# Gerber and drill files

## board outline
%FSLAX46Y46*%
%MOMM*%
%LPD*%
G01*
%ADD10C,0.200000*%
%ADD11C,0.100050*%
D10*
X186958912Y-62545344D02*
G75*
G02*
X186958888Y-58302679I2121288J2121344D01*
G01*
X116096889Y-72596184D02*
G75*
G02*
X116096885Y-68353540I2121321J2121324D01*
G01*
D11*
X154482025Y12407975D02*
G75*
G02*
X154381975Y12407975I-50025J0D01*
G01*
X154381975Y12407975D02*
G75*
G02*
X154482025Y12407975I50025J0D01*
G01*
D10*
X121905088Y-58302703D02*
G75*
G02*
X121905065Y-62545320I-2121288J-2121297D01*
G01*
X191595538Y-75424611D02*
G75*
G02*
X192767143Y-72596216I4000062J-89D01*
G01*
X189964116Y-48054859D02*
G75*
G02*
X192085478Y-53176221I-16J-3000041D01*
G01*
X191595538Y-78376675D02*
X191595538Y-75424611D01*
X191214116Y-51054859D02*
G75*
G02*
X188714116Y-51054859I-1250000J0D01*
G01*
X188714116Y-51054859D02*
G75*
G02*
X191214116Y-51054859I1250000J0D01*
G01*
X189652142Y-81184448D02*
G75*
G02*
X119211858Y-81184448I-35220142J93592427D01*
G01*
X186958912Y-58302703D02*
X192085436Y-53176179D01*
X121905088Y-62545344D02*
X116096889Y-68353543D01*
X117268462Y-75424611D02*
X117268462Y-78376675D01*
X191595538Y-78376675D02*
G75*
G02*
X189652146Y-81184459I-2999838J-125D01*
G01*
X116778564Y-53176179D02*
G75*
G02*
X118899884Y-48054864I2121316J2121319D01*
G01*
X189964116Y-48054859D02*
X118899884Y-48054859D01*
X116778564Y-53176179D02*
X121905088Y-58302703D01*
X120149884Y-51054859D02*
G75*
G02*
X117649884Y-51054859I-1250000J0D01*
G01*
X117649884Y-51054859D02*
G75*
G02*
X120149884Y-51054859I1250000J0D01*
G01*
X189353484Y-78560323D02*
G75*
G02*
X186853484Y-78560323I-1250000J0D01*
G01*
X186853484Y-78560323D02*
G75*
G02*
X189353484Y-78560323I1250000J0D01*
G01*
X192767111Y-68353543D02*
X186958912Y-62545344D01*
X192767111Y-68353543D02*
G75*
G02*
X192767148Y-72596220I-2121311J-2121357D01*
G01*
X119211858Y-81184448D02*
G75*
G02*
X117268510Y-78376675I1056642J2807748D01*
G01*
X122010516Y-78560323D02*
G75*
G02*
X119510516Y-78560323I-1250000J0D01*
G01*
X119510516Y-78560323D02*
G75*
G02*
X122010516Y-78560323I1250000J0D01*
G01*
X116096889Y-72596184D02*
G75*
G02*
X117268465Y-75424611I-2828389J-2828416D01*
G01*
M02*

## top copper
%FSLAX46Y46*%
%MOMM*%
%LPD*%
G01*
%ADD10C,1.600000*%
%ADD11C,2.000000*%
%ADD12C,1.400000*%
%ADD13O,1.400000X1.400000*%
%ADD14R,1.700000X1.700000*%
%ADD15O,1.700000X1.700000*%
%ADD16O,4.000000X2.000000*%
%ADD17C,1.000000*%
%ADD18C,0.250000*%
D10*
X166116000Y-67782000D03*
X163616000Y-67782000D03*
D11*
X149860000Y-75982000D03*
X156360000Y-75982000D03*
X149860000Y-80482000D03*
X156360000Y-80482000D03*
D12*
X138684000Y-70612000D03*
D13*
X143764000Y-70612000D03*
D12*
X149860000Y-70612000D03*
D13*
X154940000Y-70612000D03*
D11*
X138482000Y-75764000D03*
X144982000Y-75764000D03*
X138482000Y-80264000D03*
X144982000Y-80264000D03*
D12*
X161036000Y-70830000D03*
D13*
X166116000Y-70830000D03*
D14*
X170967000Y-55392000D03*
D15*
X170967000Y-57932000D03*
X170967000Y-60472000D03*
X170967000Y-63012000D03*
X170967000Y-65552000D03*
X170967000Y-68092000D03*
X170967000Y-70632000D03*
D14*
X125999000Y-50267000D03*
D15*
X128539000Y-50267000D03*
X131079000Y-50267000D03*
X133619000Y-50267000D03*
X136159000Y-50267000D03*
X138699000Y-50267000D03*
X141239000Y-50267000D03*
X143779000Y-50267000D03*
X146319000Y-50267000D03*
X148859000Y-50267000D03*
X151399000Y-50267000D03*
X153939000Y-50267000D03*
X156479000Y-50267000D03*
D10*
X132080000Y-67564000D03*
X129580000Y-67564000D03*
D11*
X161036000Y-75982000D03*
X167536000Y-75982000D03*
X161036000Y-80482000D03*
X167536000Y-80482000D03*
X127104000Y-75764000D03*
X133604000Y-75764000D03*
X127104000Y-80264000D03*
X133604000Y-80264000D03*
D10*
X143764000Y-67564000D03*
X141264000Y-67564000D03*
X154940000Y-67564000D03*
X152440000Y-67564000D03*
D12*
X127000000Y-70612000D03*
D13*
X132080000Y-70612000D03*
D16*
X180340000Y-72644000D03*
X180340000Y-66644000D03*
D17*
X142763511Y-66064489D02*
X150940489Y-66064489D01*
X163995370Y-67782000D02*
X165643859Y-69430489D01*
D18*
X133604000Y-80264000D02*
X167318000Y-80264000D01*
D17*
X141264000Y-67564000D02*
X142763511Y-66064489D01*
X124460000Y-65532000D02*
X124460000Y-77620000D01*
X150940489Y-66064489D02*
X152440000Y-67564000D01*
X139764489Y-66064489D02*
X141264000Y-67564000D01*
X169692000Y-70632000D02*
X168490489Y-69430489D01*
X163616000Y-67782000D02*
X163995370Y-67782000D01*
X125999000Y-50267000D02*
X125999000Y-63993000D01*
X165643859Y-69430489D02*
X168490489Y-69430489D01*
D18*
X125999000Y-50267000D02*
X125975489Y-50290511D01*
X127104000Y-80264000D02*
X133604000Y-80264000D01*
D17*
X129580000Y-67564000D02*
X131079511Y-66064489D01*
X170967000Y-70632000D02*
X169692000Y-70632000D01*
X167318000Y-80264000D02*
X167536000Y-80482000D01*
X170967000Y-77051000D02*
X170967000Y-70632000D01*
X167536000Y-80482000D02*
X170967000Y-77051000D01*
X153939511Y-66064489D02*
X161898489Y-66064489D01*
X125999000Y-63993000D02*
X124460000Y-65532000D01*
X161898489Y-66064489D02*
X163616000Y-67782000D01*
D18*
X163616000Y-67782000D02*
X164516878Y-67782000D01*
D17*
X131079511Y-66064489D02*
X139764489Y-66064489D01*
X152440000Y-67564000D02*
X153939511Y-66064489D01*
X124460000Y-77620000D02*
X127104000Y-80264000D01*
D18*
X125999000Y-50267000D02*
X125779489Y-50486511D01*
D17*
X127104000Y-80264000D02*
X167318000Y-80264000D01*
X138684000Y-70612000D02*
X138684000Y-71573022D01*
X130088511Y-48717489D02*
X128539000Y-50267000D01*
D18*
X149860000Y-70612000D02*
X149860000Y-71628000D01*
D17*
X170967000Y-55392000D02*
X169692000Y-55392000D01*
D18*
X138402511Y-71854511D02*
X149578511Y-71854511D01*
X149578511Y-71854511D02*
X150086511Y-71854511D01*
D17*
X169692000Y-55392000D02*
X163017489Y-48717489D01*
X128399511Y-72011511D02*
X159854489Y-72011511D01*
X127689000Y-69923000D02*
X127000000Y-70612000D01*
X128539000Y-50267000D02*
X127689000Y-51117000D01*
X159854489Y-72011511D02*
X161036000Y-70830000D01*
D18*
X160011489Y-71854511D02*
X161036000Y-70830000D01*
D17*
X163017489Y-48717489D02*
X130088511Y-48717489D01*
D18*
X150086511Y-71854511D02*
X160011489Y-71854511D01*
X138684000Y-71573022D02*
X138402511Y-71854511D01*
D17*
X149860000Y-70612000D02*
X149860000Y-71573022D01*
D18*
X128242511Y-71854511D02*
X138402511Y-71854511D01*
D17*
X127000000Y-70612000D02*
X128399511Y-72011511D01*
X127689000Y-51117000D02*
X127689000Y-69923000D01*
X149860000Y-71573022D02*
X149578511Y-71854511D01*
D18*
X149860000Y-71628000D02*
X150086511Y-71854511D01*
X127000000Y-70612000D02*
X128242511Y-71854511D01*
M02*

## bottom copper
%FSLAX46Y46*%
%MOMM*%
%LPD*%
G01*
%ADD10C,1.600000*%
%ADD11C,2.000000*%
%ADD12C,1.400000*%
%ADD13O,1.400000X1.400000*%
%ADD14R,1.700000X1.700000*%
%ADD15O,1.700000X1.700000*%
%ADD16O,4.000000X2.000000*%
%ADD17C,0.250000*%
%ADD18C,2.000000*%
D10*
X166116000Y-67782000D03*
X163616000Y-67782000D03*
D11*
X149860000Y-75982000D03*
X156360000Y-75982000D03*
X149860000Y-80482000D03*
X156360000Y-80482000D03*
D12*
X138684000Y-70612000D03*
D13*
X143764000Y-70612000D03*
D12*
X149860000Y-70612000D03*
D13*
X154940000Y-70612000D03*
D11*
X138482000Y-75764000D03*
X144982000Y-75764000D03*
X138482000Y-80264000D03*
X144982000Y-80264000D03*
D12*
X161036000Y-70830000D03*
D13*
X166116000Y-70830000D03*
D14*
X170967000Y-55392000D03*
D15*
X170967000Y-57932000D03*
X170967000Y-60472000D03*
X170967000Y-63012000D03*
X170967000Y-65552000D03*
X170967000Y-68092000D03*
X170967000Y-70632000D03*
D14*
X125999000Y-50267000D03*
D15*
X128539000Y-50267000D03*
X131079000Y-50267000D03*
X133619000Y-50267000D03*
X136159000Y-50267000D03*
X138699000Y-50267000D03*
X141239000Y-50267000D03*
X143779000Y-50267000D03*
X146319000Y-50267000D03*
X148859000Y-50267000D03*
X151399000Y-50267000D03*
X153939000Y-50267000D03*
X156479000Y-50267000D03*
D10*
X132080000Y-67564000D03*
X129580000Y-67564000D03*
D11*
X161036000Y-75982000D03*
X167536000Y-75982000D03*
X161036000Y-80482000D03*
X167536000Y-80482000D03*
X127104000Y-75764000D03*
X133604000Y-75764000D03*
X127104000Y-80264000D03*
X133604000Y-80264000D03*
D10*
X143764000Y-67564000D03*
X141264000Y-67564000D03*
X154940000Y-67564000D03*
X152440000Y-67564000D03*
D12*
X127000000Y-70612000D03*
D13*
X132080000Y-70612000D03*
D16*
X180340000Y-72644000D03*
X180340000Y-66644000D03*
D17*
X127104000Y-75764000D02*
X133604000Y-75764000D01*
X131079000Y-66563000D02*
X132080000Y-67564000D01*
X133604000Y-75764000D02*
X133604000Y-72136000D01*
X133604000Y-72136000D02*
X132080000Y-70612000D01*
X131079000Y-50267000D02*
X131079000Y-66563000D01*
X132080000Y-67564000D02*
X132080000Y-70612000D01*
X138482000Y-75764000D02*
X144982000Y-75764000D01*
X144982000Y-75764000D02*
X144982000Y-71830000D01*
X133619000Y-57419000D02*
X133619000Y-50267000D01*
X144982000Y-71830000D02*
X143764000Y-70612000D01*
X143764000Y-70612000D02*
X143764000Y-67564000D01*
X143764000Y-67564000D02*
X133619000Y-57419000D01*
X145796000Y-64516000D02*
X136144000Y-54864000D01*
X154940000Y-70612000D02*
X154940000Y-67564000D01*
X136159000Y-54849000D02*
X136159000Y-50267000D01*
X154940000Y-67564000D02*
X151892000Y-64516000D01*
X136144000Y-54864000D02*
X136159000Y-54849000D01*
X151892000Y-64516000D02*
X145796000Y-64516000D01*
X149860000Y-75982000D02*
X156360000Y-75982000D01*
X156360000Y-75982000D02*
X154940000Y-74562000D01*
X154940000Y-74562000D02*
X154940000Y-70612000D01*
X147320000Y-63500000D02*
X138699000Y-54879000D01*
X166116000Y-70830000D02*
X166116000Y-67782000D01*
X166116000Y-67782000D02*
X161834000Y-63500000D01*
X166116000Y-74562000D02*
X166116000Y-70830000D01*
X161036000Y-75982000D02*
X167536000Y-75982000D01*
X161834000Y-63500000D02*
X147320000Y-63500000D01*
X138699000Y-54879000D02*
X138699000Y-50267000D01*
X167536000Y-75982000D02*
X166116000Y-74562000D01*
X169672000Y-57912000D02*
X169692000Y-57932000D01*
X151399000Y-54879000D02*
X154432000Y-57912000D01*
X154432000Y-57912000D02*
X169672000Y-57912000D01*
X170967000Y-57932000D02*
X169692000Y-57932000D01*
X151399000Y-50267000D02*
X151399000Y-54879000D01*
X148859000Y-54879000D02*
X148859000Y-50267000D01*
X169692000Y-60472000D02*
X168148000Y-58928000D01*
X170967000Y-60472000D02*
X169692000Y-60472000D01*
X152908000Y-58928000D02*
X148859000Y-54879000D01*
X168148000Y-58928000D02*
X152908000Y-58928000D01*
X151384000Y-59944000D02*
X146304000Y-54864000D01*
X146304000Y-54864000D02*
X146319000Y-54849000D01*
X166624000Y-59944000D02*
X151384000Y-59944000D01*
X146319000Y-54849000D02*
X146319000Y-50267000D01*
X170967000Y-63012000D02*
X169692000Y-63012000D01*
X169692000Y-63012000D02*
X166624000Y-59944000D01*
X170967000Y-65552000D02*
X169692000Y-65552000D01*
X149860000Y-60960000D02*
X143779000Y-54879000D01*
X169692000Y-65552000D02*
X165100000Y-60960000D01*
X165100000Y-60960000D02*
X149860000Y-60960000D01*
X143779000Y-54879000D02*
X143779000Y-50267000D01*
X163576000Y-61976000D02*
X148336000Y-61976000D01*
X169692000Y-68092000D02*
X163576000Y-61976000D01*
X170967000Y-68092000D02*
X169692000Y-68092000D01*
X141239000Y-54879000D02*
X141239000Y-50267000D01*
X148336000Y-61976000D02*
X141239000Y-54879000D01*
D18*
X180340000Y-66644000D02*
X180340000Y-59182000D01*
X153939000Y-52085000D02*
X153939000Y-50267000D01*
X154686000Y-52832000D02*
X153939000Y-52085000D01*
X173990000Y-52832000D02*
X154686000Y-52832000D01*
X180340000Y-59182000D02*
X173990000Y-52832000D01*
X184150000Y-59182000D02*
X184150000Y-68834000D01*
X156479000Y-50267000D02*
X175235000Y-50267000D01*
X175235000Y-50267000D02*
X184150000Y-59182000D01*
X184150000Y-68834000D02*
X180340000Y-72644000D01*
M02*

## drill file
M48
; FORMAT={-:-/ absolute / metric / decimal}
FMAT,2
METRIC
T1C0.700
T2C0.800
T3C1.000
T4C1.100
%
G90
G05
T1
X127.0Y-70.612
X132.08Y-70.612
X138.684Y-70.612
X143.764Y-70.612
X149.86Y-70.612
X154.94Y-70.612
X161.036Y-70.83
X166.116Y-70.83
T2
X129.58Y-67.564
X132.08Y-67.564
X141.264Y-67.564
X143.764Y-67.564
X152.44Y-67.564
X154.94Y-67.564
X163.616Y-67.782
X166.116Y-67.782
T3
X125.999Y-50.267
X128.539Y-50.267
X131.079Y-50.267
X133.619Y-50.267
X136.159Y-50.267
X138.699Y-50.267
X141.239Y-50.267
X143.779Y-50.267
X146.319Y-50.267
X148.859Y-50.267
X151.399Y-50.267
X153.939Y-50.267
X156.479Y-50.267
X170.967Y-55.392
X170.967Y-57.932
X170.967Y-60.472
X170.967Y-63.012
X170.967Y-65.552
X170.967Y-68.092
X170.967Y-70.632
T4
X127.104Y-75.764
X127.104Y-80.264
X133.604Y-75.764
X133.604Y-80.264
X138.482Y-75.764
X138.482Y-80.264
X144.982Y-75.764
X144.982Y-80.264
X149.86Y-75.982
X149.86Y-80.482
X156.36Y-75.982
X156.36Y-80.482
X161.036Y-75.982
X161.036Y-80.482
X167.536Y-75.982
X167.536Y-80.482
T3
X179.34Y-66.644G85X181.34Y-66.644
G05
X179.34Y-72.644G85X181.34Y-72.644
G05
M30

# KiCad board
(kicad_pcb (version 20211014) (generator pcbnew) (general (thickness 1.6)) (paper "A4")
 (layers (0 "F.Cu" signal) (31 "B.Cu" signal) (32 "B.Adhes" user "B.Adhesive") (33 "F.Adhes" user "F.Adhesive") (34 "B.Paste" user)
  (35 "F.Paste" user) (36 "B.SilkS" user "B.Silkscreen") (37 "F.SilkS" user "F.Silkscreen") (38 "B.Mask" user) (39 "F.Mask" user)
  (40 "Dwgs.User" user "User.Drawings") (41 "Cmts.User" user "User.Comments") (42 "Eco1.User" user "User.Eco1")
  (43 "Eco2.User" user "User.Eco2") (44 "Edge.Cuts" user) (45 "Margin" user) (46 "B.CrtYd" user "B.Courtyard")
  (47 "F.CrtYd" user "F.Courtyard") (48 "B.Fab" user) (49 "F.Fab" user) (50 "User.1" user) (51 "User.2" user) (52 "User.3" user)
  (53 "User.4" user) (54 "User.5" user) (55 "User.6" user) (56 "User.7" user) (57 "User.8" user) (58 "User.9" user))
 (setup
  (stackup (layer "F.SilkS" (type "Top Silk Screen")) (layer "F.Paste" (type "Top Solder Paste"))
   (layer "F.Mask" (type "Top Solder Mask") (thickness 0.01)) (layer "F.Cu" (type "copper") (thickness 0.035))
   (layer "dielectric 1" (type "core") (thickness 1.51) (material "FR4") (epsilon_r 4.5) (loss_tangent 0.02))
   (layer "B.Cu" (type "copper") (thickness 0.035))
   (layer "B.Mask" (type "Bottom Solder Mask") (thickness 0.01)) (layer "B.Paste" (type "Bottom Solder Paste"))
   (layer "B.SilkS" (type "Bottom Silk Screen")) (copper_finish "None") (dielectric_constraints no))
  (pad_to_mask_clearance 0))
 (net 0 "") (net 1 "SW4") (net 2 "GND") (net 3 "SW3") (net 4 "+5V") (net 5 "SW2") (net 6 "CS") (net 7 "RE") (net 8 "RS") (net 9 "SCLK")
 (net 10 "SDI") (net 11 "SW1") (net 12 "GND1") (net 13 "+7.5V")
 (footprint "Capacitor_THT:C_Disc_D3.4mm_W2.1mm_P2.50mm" (layer "F.Cu") (at 166.116 67.782 180)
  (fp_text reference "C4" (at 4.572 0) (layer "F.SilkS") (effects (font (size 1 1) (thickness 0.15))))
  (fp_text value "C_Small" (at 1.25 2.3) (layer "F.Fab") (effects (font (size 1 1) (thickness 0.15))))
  (pad "1" thru_hole circle (at 0 0 180) (size 1.6 1.6) (drill 0.8) (layers *.Cu *.Mask) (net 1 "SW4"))
  (pad "2" thru_hole circle (at 2.5 0 180) (size 1.6 1.6) (drill 0.8) (layers *.Cu *.Mask) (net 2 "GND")))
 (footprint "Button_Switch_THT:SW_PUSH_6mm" (layer "F.Cu") (at 149.86 75.982)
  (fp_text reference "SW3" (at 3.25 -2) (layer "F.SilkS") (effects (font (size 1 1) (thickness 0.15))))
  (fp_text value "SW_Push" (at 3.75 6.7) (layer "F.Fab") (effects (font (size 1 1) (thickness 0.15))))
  (pad "1" thru_hole circle (at 0 0 90) (size 2 2) (drill 1.1) (layers *.Cu *.Mask) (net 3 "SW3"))
  (pad "1" thru_hole circle (at 6.5 0 90) (size 2 2) (drill 1.1) (layers *.Cu *.Mask) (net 3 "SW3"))
  (pad "2" thru_hole circle (at 0 4.5 90) (size 2 2) (drill 1.1) (layers *.Cu *.Mask) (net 2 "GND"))
  (pad "2" thru_hole circle (at 6.5 4.5 90) (size 2 2) (drill 1.1) (layers *.Cu *.Mask) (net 2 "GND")))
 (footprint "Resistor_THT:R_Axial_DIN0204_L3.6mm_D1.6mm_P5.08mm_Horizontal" (layer "F.Cu") (at 138.684 70.612)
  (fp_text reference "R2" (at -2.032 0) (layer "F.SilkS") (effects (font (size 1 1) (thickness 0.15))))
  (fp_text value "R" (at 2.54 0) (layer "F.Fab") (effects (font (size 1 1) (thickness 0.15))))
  (pad "1" thru_hole circle (at 0 0) (size 1.4 1.4) (drill 0.7) (layers *.Cu *.Mask) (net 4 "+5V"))
  (pad "2" thru_hole oval (at 5.08 0) (size 1.4 1.4) (drill 0.7) (layers *.Cu *.Mask) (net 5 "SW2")))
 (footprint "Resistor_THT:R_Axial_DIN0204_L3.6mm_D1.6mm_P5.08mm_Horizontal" (layer "F.Cu") (at 149.86 70.612)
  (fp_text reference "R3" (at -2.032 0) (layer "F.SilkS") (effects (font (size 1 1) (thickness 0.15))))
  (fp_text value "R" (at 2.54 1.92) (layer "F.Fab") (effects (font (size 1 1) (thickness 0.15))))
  (pad "1" thru_hole circle (at 0 0) (size 1.4 1.4) (drill 0.7) (layers *.Cu *.Mask) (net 4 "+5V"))
  (pad "2" thru_hole oval (at 5.08 0) (size 1.4 1.4) (drill 0.7) (layers *.Cu *.Mask) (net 3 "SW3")))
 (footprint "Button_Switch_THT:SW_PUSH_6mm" (layer "F.Cu") (at 138.482 75.764)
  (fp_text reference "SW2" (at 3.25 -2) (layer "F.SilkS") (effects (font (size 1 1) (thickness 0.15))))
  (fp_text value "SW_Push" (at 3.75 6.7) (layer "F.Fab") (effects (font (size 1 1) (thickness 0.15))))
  (pad "1" thru_hole circle (at 0 0 90) (size 2 2) (drill 1.1) (layers *.Cu *.Mask) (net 5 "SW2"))
  (pad "1" thru_hole circle (at 6.5 0 90) (size 2 2) (drill 1.1) (layers *.Cu *.Mask) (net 5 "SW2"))
  (pad "2" thru_hole circle (at 0 4.5 90) (size 2 2) (drill 1.1) (layers *.Cu *.Mask) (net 2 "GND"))
  (pad "2" thru_hole circle (at 6.5 4.5 90) (size 2 2) (drill 1.1) (layers *.Cu *.Mask) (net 2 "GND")))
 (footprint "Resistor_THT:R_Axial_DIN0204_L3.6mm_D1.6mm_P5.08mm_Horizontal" (layer "F.Cu") (at 161.036 70.83)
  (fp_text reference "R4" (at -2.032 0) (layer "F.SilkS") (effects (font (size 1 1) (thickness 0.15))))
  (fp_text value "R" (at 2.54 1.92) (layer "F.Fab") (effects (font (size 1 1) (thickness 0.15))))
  (pad "1" thru_hole circle (at 0 0) (size 1.4 1.4) (drill 0.7) (layers *.Cu *.Mask) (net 4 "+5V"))
  (pad "2" thru_hole oval (at 5.08 0) (size 1.4 1.4) (drill 0.7) (layers *.Cu *.Mask) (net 1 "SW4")))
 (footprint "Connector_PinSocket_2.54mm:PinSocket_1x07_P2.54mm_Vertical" (layer "F.Cu") (at 170.967 55.392)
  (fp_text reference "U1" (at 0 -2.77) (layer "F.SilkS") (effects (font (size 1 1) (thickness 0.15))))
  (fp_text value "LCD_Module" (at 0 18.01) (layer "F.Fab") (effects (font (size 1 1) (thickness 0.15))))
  (pad "1" thru_hole rect (at 0 0) (size 1.7 1.7) (drill 1) (layers *.Cu *.Mask) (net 4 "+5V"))
  (pad "2" thru_hole oval (at 0 2.54) (size 1.7 1.7) (drill 1) (layers *.Cu *.Mask) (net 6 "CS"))
  (pad "3" thru_hole oval (at 0 5.08) (size 1.7 1.7) (drill 1) (layers *.Cu *.Mask) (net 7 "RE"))
  (pad "4" thru_hole oval (at 0 7.62) (size 1.7 1.7) (drill 1) (layers *.Cu *.Mask) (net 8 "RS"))
  (pad "5" thru_hole oval (at 0 10.16) (size 1.7 1.7) (drill 1) (layers *.Cu *.Mask) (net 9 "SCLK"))
  (pad "6" thru_hole oval (at 0 12.7) (size 1.7 1.7) (drill 1) (layers *.Cu *.Mask) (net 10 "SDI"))
  (pad "7" thru_hole oval (at 0 15.24) (size 1.7 1.7) (drill 1) (layers *.Cu *.Mask) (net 2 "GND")))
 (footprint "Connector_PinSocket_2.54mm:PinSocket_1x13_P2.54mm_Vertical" (layer "F.Cu") (at 125.999 50.267 90)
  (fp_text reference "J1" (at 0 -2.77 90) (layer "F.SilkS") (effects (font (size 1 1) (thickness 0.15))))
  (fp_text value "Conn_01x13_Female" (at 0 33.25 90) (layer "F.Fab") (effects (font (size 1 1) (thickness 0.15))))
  (pad "1" thru_hole rect (at 0 0 90) (size 1.7 1.7) (drill 1) (layers *.Cu *.Mask) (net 2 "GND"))
  (pad "2" thru_hole oval (at 0 2.54 90) (size 1.7 1.7) (drill 1) (layers *.Cu *.Mask) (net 4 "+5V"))
  (pad "3" thru_hole oval (at 0 5.08 90) (size 1.7 1.7) (drill 1) (layers *.Cu *.Mask) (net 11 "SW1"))
  (pad "4" thru_hole oval (at 0 7.62 90) (size 1.7 1.7) (drill 1) (layers *.Cu *.Mask) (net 5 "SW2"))
  (pad "5" thru_hole oval (at 0 10.16 90) (size 1.7 1.7) (drill 1) (layers *.Cu *.Mask) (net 3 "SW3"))
  (pad "6" thru_hole oval (at 0 12.7 90) (size 1.7 1.7) (drill 1) (layers *.Cu *.Mask) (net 1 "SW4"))
  (pad "7" thru_hole oval (at 0 15.24 90) (size 1.7 1.7) (drill 1) (layers *.Cu *.Mask) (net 10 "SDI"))
  (pad "8" thru_hole oval (at 0 17.78 90) (size 1.7 1.7) (drill 1) (layers *.Cu *.Mask) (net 9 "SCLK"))
  (pad "9" thru_hole oval (at 0 20.32 90) (size 1.7 1.7) (drill 1) (layers *.Cu *.Mask) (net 8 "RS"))
  (pad "10" thru_hole oval (at 0 22.86 90) (size 1.7 1.7) (drill 1) (layers *.Cu *.Mask) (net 7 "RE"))
  (pad "11" thru_hole oval (at 0 25.4 90) (size 1.7 1.7) (drill 1) (layers *.Cu *.Mask) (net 6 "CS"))
  (pad "12" thru_hole oval (at 0 27.94 90) (size 1.7 1.7) (drill 1) (layers *.Cu *.Mask) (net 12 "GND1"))
  (pad "13" thru_hole oval (at 0 30.48 90) (size 1.7 1.7) (drill 1) (layers *.Cu *.Mask) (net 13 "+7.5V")))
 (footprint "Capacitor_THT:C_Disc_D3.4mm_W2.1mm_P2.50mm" (layer "F.Cu") (at 132.08 67.564 180)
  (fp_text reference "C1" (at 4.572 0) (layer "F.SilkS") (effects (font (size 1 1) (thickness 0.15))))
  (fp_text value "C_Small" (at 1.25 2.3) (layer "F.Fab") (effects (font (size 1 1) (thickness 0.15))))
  (pad "1" thru_hole circle (at 0 0 180) (size 1.6 1.6) (drill 0.8) (layers *.Cu *.Mask) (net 11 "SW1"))
  (pad "2" thru_hole circle (at 2.5 0 180) (size 1.6 1.6) (drill 0.8) (layers *.Cu *.Mask) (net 2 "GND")))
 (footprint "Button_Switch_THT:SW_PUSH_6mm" (layer "F.Cu") (at 161.036 75.982)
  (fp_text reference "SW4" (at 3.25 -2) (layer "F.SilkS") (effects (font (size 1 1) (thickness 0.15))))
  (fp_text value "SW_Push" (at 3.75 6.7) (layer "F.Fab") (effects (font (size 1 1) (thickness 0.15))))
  (pad "1" thru_hole circle (at 0 0 90) (size 2 2) (drill 1.1) (layers *.Cu *.Mask) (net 1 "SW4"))
  (pad "1" thru_hole circle (at 6.5 0 90) (size 2 2) (drill 1.1) (layers *.Cu *.Mask) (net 1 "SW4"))
  (pad "2" thru_hole circle (at 0 4.5 90) (size 2 2) (drill 1.1) (layers *.Cu *.Mask) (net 2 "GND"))
  (pad "2" thru_hole circle (at 6.5 4.5 90) (size 2 2) (drill 1.1) (layers *.Cu *.Mask) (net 2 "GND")))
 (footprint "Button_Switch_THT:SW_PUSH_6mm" (layer "F.Cu") (at 127.104 75.764)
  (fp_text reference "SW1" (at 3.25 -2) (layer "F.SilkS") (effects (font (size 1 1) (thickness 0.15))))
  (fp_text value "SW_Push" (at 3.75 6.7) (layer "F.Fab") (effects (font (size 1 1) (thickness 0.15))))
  (pad "1" thru_hole circle (at 0 0 90) (size 2 2) (drill 1.1) (layers *.Cu *.Mask) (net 11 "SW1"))
  (pad "1" thru_hole circle (at 6.5 0 90) (size 2 2) (drill 1.1) (layers *.Cu *.Mask) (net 11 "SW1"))
  (pad "2" thru_hole circle (at 0 4.5 90) (size 2 2) (drill 1.1) (layers *.Cu *.Mask) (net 2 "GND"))
  (pad "2" thru_hole circle (at 6.5 4.5 90) (size 2 2) (drill 1.1) (layers *.Cu *.Mask) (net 2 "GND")))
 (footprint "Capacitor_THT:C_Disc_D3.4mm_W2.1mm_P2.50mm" (layer "F.Cu") (at 143.764 67.564 180)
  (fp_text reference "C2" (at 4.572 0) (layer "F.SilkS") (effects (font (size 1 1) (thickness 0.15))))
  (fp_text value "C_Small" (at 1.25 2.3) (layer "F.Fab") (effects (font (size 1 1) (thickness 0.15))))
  (pad "1" thru_hole circle (at 0 0 180) (size 1.6 1.6) (drill 0.8) (layers *.Cu *.Mask) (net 5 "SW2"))
  (pad "2" thru_hole circle (at 2.5 0 180) (size 1.6 1.6) (drill 0.8) (layers *.Cu *.Mask) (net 2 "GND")))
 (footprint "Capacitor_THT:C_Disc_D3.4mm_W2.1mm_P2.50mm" (layer "F.Cu") (at 154.94 67.564 180)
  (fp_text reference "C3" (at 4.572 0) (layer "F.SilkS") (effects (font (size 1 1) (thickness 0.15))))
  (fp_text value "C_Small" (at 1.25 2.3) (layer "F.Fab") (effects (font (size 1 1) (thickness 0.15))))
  (pad "1" thru_hole circle (at 0 0 180) (size 1.6 1.6) (drill 0.8) (layers *.Cu *.Mask) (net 3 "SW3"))
  (pad "2" thru_hole circle (at 2.5 0 180) (size 1.6 1.6) (drill 0.8) (layers *.Cu *.Mask) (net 2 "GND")))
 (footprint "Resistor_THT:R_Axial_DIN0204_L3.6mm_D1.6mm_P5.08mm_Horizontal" (layer "F.Cu") (at 127 70.612)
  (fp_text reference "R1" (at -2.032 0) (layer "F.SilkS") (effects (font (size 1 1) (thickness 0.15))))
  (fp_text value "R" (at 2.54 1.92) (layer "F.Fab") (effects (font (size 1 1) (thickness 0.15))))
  (pad "1" thru_hole circle (at 0 0) (size 1.4 1.4) (drill 0.7) (layers *.Cu *.Mask) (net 4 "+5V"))
  (pad "2" thru_hole oval (at 5.08 0) (size 1.4 1.4) (drill 0.7) (layers *.Cu *.Mask) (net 11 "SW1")))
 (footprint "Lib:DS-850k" (layer "F.Cu") (at 180.34 72.644 -90)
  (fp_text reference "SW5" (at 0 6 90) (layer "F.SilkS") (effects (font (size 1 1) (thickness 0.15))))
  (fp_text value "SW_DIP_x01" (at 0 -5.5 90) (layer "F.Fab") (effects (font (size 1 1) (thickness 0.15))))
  (pad "1" thru_hole oval locked (at 0 0) (size 4 2) (drill oval 3 1) (layers *.Cu *.Mask) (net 13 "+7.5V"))
  (pad "2" thru_hole oval locked (at -6 0) (size 4 2) (drill oval 3 1) (layers *.Cu *.Mask) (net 12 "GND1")))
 (gr_arc (start 186.958912 62.545344) (mid 186.080233 60.424024) (end 186.958912 58.302703) (layer "Edge.Cuts") (width 0.2))
 (gr_arc (start 116.096889 72.596184) (mid 115.218209 70.474864) (end 116.096889 68.353543) (layer "Edge.Cuts") (width 0.2))
 (gr_circle (center 154.432 -12.407975) (end 154.532 -12.407975) (layer "Edge.Cuts") (width 0.0001) (fill solid))
 (gr_arc (start 121.905088 58.302703) (mid 122.783768 60.424024) (end 121.905088 62.545344) (layer "Edge.Cuts") (width 0.2))
 (gr_arc (start 191.595538 75.424611) (mid 191.900027 73.893882) (end 192.767111 72.596184) (layer "Edge.Cuts") (width 0.2))
 (gr_arc (start 189.964116 48.054859) (mid 192.735755 49.906807) (end 192.085436 53.176179) (layer "Edge.Cuts") (width 0.2))
 (gr_line (start 191.595538 78.376675) (end 191.595538 75.424611) (layer "Edge.Cuts") (width 0.2))
 (gr_circle (center 189.964116 51.054859) (end 191.214116 51.054859) (layer "Edge.Cuts") (width 0.2) (fill none))
 (gr_arc (start 189.652142 81.184448) (mid 154.432 87.592025) (end 119.211858 81.184448) (layer "Edge.Cuts") (width 0.2))
 (gr_line (start 186.958912 58.302703) (end 192.085436 53.176179) (layer "Edge.Cuts") (width 0.2))
 (gr_line (start 121.905088 62.545344) (end 116.096889 68.353543) (layer "Edge.Cuts") (width 0.2))
 (gr_line (start 117.268462 75.424611) (end 117.268462 78.376675) (layer "Edge.Cuts") (width 0.2))
 (gr_arc (start 191.595538 78.376675) (mid 191.062321 80.084069) (end 189.652142 81.184448) (layer "Edge.Cuts") (width 0.2))
 (gr_arc (start 116.778564 53.176179) (mid 116.128246 49.906809) (end 118.899884 48.054859) (layer "Edge.Cuts") (width 0.2))
 (gr_line (start 189.964116 48.054859) (end 118.899884 48.054859) (layer "Edge.Cuts") (width 0.2))
 (gr_line (start 116.778564 53.176179) (end 121.905088 58.302703) (layer "Edge.Cuts") (width 0.2))
 (gr_circle (center 118.899884 51.054859) (end 120.149884 51.054859) (layer "Edge.Cuts") (width 0.2) (fill none))
 (gr_circle (center 188.103484 78.560323) (end 189.353484 78.560323) (layer "Edge.Cuts") (width 0.2) (fill none))
 (gr_line (start 192.767111 68.353543) (end 186.958912 62.545344) (layer "Edge.Cuts") (width 0.2))
 (gr_arc (start 192.767111 68.353543) (mid 193.645792 70.474864) (end 192.767111 72.596184) (layer "Edge.Cuts") (width 0.2))
 (gr_arc (start 119.211858 81.184448) (mid 117.801702 80.08404) (end 117.268462 78.376675) (layer "Edge.Cuts") (width 0.2))
 (gr_circle (center 120.760516 78.560323) (end 122.010516 78.560323) (layer "Edge.Cuts") (width 0.2) (fill none))
 (gr_arc (start 116.096889 72.596184) (mid 116.96398 73.893877) (end 117.268462 75.424611) (layer "Edge.Cuts") (width 0.2))
 (segment (start 127.104 75.764) (end 133.604 75.764) (width 0.25) (layer "B.Cu") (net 11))
 (segment (start 131.079 66.563) (end 132.08 67.564) (width 0.25) (layer "B.Cu") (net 11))
 (segment (start 133.604 75.764) (end 133.604 72.136) (width 0.25) (layer "B.Cu") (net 11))
 (segment (start 133.604 72.136) (end 132.08 70.612) (width 0.25) (layer "B.Cu") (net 11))
 (segment (start 131.079 50.267) (end 131.079 66.563) (width 0.25) (layer "B.Cu") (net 11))
 (segment (start 132.08 67.564) (end 132.08 70.612) (width 0.25) (layer "B.Cu") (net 11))
 (segment (start 142.763511 66.064489) (end 150.940489 66.064489) (width 1) (layer "F.Cu") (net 2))
 (segment (start 163.99537 67.782) (end 165.643859 69.430489) (width 1) (layer "F.Cu") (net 2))
 (segment (start 133.604 80.264) (end 167.318 80.264) (width 0.25) (layer "F.Cu") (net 2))
 (segment (start 141.264 67.564) (end 142.763511 66.064489) (width 1) (layer "F.Cu") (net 2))
 (segment (start 124.46 65.532) (end 124.46 77.62) (width 1) (layer "F.Cu") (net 2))
 (segment (start 150.940489 66.064489) (end 152.44 67.564) (width 1) (layer "F.Cu") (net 2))
 (segment (start 139.764489 66.064489) (end 141.264 67.564) (width 1) (layer "F.Cu") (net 2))
 (segment (start 169.692 70.632) (end 168.490489 69.430489) (width 1) (layer "F.Cu") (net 2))
 (segment (start 163.616 67.782) (end 163.99537 67.782) (width 1) (layer "F.Cu") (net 2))
 (segment (start 125.999 50.267) (end 125.999 63.993) (width 1) (layer "F.Cu") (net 2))
 (segment (start 165.643859 69.430489) (end 168.490489 69.430489) (width 1) (layer "F.Cu") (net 2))
 (segment (start 125.999 50.267) (end 125.975489 50.290511) (width 0.25) (layer "F.Cu") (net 2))
 (segment (start 127.104 80.264) (end 133.604 80.264) (width 0.25) (layer "F.Cu") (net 2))
 (segment (start 129.58 67.564) (end 131.079511 66.064489) (width 1) (layer "F.Cu") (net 2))
 (segment (start 170.967 70.632) (end 169.692 70.632) (width 1) (layer "F.Cu") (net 2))
 (segment (start 167.318 80.264) (end 167.536 80.482) (width 1) (layer "F.Cu") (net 2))
 (segment (start 170.967 77.051) (end 170.967 70.632) (width 1) (layer "F.Cu") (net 2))
 (segment (start 167.536 80.482) (end 170.967 77.051) (width 1) (layer "F.Cu") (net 2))
 (segment (start 153.939511 66.064489) (end 161.898489 66.064489) (width 1) (layer "F.Cu") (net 2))
 (segment (start 125.999 63.993) (end 124.46 65.532) (width 1) (layer "F.Cu") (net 2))
 (segment (start 161.898489 66.064489) (end 163.616 67.782) (width 1) (layer "F.Cu") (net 2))
 (segment (start 163.616 67.782) (end 164.516878 67.782) (width 0.25) (layer "F.Cu") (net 2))
 (segment (start 131.079511 66.064489) (end 139.764489 66.064489) (width 1) (layer "F.Cu") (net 2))
 (segment (start 152.44 67.564) (end 153.939511 66.064489) (width 1) (layer "F.Cu") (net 2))
 (segment (start 124.46 77.62) (end 127.104 80.264) (width 1) (layer "F.Cu") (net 2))
 (segment (start 125.999 50.267) (end 125.779489 50.486511) (width 0.25) (layer "F.Cu") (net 2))
 (segment (start 127.104 80.264) (end 167.318 80.264) (width 1) (layer "F.Cu") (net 2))
 (segment (start 138.482 75.764) (end 144.982 75.764) (width 0.25) (layer "B.Cu") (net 5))
 (segment (start 144.982 75.764) (end 144.982 71.83) (width 0.25) (layer "B.Cu") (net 5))
 (segment (start 133.619 57.419) (end 133.619 50.267) (width 0.25) (layer "B.Cu") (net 5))
 (segment (start 144.982 71.83) (end 143.764 70.612) (width 0.25) (layer "B.Cu") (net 5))
 (segment (start 143.764 70.612) (end 143.764 67.564) (width 0.25) (layer "B.Cu") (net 5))
 (segment (start 143.764 67.564) (end 133.619 57.419) (width 0.25) (layer "B.Cu") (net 5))
 (segment (start 145.796 64.516) (end 136.144 54.864) (width 0.25) (layer "B.Cu") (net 3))
 (segment (start 154.94 70.612) (end 154.94 67.564) (width 0.25) (layer "B.Cu") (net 3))
 (segment (start 136.159 54.849) (end 136.159 50.267) (width 0.25) (layer "B.Cu") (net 3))
 (segment (start 154.94 67.564) (end 151.892 64.516) (width 0.25) (layer "B.Cu") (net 3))
 (segment (start 136.144 54.864) (end 136.159 54.849) (width 0.25) (layer "B.Cu") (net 3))
 (segment (start 151.892 64.516) (end 145.796 64.516) (width 0.25) (layer "B.Cu") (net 3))
 (segment (start 149.86 75.982) (end 156.36 75.982) (width 0.25) (layer "B.Cu") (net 3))
 (segment (start 156.36 75.982) (end 154.94 74.562) (width 0.25) (layer "B.Cu") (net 3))
 (segment (start 154.94 74.562) (end 154.94 70.612) (width 0.25) (layer "B.Cu") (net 3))
 (segment (start 147.32 63.5) (end 138.699 54.879) (width 0.25) (layer "B.Cu") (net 1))
 (segment (start 166.116 70.83) (end 166.116 67.782) (width 0.25) (layer "B.Cu") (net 1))
 (segment (start 166.116 67.782) (end 161.834 63.5) (width 0.25) (layer "B.Cu") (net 1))
 (segment (start 166.116 74.562) (end 166.116 70.83) (width 0.25) (layer "B.Cu") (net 1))
 (segment (start 161.036 75.982) (end 167.536 75.982) (width 0.25) (layer "B.Cu") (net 1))
 (segment (start 161.834 63.5) (end 147.32 63.5) (width 0.25) (layer "B.Cu") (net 1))
 (segment (start 138.699 54.879) (end 138.699 50.267) (width 0.25) (layer "B.Cu") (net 1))
 (segment (start 167.536 75.982) (end 166.116 74.562) (width 0.25) (layer "B.Cu") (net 1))
 (segment (start 138.684 70.612) (end 138.684 71.573022) (width 1) (layer "F.Cu") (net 4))
 (segment (start 130.088511 48.717489) (end 128.539 50.267) (width 1) (layer "F.Cu") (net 4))
 (segment (start 149.86 70.612) (end 149.86 71.628) (width 0.25) (layer "F.Cu") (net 4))
 (segment (start 170.967 55.392) (end 169.692 55.392) (width 1) (layer "F.Cu") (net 4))
 (segment (start 138.402511 71.854511) (end 149.578511 71.854511) (width 0.25) (layer "F.Cu") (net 4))
 (segment (start 149.578511 71.854511) (end 150.086511 71.854511) (width 0.25) (layer "F.Cu") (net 4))
 (segment (start 169.692 55.392) (end 163.017489 48.717489) (width 1) (layer "F.Cu") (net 4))
 (segment (start 128.399511 72.011511) (end 159.854489 72.011511) (width 1) (layer "F.Cu") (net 4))
 (segment (start 127.689 69.923) (end 127 70.612) (width 1) (layer "F.Cu") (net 4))
 (segment (start 128.539 50.267) (end 127.689 51.117) (width 1) (layer "F.Cu") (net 4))
 (segment (start 159.854489 72.011511) (end 161.036 70.83) (width 1) (layer "F.Cu") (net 4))
 (segment (start 160.011489 71.854511) (end 161.036 70.83) (width 0.25) (layer "F.Cu") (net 4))
 (segment (start 163.017489 48.717489) (end 130.088511 48.717489) (width 1) (layer "F.Cu") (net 4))
 (segment (start 150.086511 71.854511) (end 160.011489 71.854511) (width 0.25) (layer "F.Cu") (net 4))
 (segment (start 138.684 71.573022) (end 138.402511 71.854511) (width 0.25) (layer "F.Cu") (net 4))
 (segment (start 149.86 70.612) (end 149.86 71.573022) (width 1) (layer "F.Cu") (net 4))
 (segment (start 128.242511 71.854511) (end 138.402511 71.854511) (width 0.25) (layer "F.Cu") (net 4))
 (segment (start 127 70.612) (end 128.399511 72.011511) (width 1) (layer "F.Cu") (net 4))
 (segment (start 127.689 51.117) (end 127.689 69.923) (width 1) (layer "F.Cu") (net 4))
 (segment (start 149.86 71.573022) (end 149.578511 71.854511) (width 1) (layer "F.Cu") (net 4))
 (segment (start 149.86 71.628) (end 150.086511 71.854511) (width 0.25) (layer "F.Cu") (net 4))
 (segment (start 127 70.612) (end 128.242511 71.854511) (width 0.25) (layer "F.Cu") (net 4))
 (segment (start 169.672 57.912) (end 169.692 57.932) (width 0.25) (layer "B.Cu") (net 6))
 (segment (start 151.399 54.879) (end 154.432 57.912) (width 0.25) (layer "B.Cu") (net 6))
 (segment (start 154.432 57.912) (end 169.672 57.912) (width 0.25) (layer "B.Cu") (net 6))
 (segment (start 170.967 57.932) (end 169.692 57.932) (width 0.25) (layer "B.Cu") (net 6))
 (segment (start 151.399 50.267) (end 151.399 54.879) (width 0.25) (layer "B.Cu") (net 6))
 (segment (start 148.859 54.879) (end 148.859 50.267) (width 0.25) (layer "B.Cu") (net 7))
 (segment (start 169.692 60.472) (end 168.148 58.928) (width 0.25) (layer "B.Cu") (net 7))
 (segment (start 170.967 60.472) (end 169.692 60.472) (width 0.25) (layer "B.Cu") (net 7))
 (segment (start 152.908 58.928) (end 148.859 54.879) (width 0.25) (layer "B.Cu") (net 7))
 (segment (start 168.148 58.928) (end 152.908 58.928) (width 0.25) (layer "B.Cu") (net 7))
 (segment (start 151.384 59.944) (end 146.304 54.864) (width 0.25) (layer "B.Cu") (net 8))
 (segment (start 146.304 54.864) (end 146.319 54.849) (width 0.25) (layer "B.Cu") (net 8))
 (segment (start 166.624 59.944) (end 151.384 59.944) (width 0.25) (layer "B.Cu") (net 8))
 (segment (start 146.319 54.849) (end 146.319 50.267) (width 0.25) (layer "B.Cu") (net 8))
 (segment (start 170.967 63.012) (end 169.692 63.012) (width 0.25) (layer "B.Cu") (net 8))
 (segment (start 169.692 63.012) (end 166.624 59.944) (width 0.25) (layer "B.Cu") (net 8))
 (segment (start 170.967 65.552) (end 169.692 65.552) (width 0.25) (layer "B.Cu") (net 9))
 (segment (start 149.86 60.96) (end 143.779 54.879) (width 0.25) (layer "B.Cu") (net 9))
 (segment (start 169.692 65.552) (end 165.1 60.96) (width 0.25) (layer "B.Cu") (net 9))
 (segment (start 165.1 60.96) (end 149.86 60.96) (width 0.25) (layer "B.Cu") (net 9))
 (segment (start 143.779 54.879) (end 143.779 50.267) (width 0.25) (layer "B.Cu") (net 9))
 (segment (start 163.576 61.976) (end 148.336 61.976) (width 0.25) (layer "B.Cu") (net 10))
 (segment (start 169.692 68.092) (end 163.576 61.976) (width 0.25) (layer "B.Cu") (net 10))
 (segment (start 170.967 68.092) (end 169.692 68.092) (width 0.25) (layer "B.Cu") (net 10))
 (segment (start 141.239 54.879) (end 141.239 50.267) (width 0.25) (layer "B.Cu") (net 10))
 (segment (start 148.336 61.976) (end 141.239 54.879) (width 0.25) (layer "B.Cu") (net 10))
 (segment (start 180.34 66.644) (end 180.34 59.182) (width 2) (layer "B.Cu") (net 12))
 (segment (start 153.939 52.085) (end 153.939 50.267) (width 2) (layer "B.Cu") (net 12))
 (segment (start 154.686 52.832) (end 153.939 52.085) (width 2) (layer "B.Cu") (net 12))
 (segment (start 173.99 52.832) (end 154.686 52.832) (width 2) (layer "B.Cu") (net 12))
 (segment (start 180.34 59.182) (end 173.99 52.832) (width 2) (layer "B.Cu") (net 12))
 (segment (start 184.15 59.182) (end 184.15 68.834) (width 2) (layer "B.Cu") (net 13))
 (segment (start 156.479 50.267) (end 175.235 50.267) (width 2) (layer "B.Cu") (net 13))
 (segment (start 175.235 50.267) (end 184.15 59.182) (width 2) (layer "B.Cu") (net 13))
 (segment (start 184.15 68.834) (end 180.34 72.644) (width 2) (layer "B.Cu") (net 13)))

